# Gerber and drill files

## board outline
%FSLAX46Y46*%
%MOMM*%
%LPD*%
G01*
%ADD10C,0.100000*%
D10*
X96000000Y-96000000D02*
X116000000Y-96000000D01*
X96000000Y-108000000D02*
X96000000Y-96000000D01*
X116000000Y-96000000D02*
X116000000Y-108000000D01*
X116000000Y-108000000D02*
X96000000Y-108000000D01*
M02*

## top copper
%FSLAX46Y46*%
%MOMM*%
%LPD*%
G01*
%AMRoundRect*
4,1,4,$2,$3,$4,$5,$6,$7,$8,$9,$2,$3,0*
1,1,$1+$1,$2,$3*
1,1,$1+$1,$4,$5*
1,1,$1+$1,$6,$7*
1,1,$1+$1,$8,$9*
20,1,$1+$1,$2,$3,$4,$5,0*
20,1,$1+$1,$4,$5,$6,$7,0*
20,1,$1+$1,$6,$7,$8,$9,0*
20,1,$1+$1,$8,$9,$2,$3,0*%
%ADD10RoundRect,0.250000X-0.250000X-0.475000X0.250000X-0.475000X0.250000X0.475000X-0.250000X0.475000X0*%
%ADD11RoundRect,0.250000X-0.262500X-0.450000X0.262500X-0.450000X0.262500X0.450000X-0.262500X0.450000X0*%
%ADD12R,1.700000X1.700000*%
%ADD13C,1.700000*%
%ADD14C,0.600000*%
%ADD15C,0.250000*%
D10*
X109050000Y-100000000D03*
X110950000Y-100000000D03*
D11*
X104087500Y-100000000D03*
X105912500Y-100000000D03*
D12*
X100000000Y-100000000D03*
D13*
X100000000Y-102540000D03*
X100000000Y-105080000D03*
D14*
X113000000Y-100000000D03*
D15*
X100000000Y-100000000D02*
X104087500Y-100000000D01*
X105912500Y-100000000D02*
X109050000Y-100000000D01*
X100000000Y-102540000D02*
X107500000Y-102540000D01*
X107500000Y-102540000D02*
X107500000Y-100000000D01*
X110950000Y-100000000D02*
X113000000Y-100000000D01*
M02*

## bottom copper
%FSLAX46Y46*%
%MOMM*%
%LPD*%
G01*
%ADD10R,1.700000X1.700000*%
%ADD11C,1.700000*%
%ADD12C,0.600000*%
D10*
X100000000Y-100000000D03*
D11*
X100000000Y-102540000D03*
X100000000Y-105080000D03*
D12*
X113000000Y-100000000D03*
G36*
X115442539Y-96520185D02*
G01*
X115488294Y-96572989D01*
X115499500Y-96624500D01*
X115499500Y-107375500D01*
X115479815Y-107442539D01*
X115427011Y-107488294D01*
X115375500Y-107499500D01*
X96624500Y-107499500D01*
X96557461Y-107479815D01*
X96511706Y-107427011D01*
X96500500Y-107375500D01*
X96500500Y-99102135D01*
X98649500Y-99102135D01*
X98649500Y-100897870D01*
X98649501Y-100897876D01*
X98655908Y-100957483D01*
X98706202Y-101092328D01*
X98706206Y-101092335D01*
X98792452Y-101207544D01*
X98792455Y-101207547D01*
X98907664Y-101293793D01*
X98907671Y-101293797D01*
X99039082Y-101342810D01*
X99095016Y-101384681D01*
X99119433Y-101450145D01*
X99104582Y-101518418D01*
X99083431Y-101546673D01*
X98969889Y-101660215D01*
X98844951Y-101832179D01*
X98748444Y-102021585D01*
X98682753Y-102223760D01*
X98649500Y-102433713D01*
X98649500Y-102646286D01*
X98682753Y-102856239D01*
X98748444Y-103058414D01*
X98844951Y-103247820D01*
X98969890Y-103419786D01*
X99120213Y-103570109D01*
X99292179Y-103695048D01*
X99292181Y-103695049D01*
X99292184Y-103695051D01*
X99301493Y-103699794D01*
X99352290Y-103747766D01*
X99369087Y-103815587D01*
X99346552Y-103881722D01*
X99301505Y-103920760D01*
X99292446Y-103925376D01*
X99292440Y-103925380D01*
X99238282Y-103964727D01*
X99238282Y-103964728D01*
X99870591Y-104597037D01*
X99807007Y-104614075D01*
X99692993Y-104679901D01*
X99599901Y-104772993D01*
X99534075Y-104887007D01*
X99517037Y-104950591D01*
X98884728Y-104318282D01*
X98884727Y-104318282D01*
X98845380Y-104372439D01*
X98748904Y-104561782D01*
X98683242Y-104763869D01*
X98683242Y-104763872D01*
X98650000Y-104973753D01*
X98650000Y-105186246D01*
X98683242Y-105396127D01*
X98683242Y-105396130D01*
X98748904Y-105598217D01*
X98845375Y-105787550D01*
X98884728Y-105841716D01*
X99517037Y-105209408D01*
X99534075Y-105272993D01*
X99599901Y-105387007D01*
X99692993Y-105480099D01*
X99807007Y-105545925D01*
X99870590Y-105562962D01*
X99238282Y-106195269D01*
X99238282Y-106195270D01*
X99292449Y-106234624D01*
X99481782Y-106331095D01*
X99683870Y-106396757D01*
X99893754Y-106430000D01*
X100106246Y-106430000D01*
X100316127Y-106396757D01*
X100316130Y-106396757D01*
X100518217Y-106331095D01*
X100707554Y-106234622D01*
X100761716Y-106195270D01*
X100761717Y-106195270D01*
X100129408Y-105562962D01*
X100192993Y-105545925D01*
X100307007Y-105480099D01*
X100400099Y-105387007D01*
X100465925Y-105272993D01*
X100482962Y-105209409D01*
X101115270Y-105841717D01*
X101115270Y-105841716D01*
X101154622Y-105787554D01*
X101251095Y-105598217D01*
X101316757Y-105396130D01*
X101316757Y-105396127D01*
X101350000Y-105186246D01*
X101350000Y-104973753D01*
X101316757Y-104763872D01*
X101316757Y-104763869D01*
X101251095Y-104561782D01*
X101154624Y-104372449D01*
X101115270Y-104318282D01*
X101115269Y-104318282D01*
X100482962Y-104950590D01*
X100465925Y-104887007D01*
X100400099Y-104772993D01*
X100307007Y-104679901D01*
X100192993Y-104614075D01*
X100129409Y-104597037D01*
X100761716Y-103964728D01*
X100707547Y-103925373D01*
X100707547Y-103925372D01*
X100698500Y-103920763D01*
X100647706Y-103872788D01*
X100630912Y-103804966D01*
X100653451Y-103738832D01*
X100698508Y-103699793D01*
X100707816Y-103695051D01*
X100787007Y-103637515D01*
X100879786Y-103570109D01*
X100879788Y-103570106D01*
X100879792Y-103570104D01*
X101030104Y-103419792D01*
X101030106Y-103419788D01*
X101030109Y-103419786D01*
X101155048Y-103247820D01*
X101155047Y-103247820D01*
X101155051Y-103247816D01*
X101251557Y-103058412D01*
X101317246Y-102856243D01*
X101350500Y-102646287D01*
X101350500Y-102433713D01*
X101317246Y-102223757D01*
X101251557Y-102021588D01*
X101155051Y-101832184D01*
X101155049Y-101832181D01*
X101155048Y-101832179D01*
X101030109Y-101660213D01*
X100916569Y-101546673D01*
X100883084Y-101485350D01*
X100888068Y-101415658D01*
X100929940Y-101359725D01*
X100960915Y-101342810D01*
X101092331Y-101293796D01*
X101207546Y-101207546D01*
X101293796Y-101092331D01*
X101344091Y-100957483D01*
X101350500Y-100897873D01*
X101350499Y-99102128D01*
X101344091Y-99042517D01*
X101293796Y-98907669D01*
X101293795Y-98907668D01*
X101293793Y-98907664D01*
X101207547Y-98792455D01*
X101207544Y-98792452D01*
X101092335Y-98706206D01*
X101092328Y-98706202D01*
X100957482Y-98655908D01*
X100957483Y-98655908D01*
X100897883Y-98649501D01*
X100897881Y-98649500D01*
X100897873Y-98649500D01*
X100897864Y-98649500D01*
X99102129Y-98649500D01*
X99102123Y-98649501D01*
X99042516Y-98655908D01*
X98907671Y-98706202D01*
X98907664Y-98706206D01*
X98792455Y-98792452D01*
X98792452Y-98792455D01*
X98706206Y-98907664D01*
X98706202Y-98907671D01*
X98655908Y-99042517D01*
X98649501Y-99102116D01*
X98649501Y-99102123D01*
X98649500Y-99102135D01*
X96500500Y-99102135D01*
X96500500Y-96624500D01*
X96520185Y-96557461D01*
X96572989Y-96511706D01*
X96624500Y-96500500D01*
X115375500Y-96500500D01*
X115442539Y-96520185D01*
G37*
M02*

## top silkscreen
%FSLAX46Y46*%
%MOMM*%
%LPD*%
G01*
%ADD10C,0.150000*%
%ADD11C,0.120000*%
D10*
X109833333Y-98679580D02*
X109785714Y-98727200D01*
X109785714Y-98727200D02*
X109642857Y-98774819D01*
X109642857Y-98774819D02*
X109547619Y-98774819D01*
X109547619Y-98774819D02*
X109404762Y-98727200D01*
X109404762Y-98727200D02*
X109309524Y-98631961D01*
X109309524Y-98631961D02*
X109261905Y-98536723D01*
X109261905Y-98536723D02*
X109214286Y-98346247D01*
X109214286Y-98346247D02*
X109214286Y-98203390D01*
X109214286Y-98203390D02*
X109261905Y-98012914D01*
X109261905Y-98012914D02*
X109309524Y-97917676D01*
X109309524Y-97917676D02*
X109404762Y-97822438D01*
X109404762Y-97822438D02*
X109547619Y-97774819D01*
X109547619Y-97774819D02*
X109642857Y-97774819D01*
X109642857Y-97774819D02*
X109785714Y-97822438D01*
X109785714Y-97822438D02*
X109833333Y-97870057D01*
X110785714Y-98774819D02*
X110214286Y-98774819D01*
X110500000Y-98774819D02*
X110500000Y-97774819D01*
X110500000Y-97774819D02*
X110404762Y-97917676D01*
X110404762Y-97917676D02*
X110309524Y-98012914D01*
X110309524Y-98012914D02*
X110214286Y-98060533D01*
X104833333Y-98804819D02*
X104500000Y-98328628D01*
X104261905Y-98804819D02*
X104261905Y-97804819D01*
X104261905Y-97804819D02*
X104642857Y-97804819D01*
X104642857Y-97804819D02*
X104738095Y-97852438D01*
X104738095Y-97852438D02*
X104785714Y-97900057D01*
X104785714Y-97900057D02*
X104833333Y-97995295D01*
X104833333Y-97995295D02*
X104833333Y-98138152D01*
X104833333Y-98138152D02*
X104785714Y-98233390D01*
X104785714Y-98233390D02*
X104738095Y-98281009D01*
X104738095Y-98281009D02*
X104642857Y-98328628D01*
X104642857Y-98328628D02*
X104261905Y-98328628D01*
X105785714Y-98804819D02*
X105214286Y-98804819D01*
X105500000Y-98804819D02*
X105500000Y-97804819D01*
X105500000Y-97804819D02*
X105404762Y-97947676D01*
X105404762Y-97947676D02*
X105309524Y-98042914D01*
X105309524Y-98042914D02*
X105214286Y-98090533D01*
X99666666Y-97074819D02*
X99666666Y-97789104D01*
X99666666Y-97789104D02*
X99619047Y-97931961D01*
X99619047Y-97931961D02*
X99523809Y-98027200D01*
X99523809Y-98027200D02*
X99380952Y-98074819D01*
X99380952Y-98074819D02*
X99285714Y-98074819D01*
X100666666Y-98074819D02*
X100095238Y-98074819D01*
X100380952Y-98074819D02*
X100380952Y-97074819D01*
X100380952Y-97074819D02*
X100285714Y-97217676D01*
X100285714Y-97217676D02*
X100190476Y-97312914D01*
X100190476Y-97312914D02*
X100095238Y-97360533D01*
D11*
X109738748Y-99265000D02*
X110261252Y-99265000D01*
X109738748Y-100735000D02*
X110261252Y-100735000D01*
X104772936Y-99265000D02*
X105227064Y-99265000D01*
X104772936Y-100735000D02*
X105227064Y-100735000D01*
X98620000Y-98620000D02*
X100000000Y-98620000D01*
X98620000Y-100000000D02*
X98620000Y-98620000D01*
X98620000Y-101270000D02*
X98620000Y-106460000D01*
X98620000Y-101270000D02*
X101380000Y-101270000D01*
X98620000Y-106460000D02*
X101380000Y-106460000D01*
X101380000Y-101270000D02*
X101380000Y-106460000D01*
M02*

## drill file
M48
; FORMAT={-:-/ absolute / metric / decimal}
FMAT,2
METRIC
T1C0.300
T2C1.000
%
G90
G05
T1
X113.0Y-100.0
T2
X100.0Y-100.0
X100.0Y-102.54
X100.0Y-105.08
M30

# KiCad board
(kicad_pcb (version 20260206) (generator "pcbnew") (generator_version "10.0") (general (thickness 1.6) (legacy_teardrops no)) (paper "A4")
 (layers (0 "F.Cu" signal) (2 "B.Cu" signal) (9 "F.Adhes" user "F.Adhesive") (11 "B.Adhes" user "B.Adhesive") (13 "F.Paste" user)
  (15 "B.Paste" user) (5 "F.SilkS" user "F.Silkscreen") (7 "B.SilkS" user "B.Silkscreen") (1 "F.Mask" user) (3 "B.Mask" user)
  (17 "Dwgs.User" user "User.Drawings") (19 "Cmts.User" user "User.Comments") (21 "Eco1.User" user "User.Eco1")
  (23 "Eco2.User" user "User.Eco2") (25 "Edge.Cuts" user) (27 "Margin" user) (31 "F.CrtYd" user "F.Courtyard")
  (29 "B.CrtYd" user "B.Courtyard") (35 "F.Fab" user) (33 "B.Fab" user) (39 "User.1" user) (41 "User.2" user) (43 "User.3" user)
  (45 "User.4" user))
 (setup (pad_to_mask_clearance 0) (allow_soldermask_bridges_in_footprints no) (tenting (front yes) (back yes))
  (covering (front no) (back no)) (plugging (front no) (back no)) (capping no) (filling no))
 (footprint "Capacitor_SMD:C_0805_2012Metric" (layer "F.Cu") (at 110 100)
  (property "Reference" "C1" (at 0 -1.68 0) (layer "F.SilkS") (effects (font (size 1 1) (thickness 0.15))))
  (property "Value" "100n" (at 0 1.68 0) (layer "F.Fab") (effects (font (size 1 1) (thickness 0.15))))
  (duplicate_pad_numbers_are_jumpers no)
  (fp_line (start -0.261252 -0.735) (end 0.261252 -0.735) (stroke (width 0.12) (type solid)) (layer "F.SilkS"))
  (fp_line (start -0.261252 0.735) (end 0.261252 0.735) (stroke (width 0.12) (type solid)) (layer "F.SilkS"))
  (pad "1" smd roundrect (at -0.95 0) (size 1 1.45) (layers "F.Cu" "F.Mask" "F.Paste") (roundrect_rratio 0.25) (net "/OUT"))
  (pad "2" smd roundrect (at 0.95 0) (size 1 1.45) (layers "F.Cu" "F.Mask" "F.Paste") (roundrect_rratio 0.25) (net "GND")))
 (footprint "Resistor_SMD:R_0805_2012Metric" (layer "F.Cu") (at 105 100)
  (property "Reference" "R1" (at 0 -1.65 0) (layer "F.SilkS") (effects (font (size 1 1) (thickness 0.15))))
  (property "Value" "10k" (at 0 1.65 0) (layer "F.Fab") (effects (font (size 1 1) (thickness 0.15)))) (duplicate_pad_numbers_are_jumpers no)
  (fp_line (start -0.227064 -0.735) (end 0.227064 -0.735) (stroke (width 0.12) (type solid)) (layer "F.SilkS"))
  (fp_line (start -0.227064 0.735) (end 0.227064 0.735) (stroke (width 0.12) (type solid)) (layer "F.SilkS"))
  (pad "1" smd roundrect (at -0.9125 0) (size 1.025 1.4) (layers "F.Cu" "F.Mask" "F.Paste") (roundrect_rratio 0.243902) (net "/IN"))
  (pad "2" smd roundrect (at 0.9125 0) (size 1.025 1.4) (layers "F.Cu" "F.Mask" "F.Paste") (roundrect_rratio 0.243902) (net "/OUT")))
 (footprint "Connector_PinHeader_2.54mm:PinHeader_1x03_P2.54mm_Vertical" (layer "F.Cu") (at 100 100)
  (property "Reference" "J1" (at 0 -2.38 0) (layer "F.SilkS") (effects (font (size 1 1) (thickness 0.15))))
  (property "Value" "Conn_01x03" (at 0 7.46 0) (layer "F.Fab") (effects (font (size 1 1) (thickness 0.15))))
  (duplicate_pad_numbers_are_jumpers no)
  (fp_line (start -1.38 -1.38) (end 0 -1.38) (stroke (width 0.12) (type solid)) (layer "F.SilkS"))
  (fp_line (start -1.38 0) (end -1.38 -1.38) (stroke (width 0.12) (type solid)) (layer "F.SilkS"))
  (fp_line (start -1.38 1.27) (end -1.38 6.46) (stroke (width 0.12) (type solid)) (layer "F.SilkS"))
  (fp_line (start -1.38 1.27) (end 1.38 1.27) (stroke (width 0.12) (type solid)) (layer "F.SilkS"))
  (fp_line (start -1.38 6.46) (end 1.38 6.46) (stroke (width 0.12) (type solid)) (layer "F.SilkS"))
  (fp_line (start 1.38 1.27) (end 1.38 6.46) (stroke (width 0.12) (type solid)) (layer "F.SilkS"))
  (pad "1" thru_hole rect (at 0 0) (size 1.7 1.7) (drill 1) (layers "*.Cu" "*.Mask") (remove_unused_layers no) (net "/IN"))
  (pad "2" thru_hole circle (at 0 2.54) (size 1.7 1.7) (drill 1) (layers "*.Cu" "*.Mask") (remove_unused_layers no) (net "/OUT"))
  (pad "3" thru_hole circle (at 0 5.08) (size 1.7 1.7) (drill 1) (layers "*.Cu" "*.Mask") (remove_unused_layers no) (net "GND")))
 (gr_line (start 96 96) (end 116 96) (stroke (width 0.1) (type default)) (layer "Edge.Cuts"))
 (gr_line (start 96 108) (end 96 96) (stroke (width 0.1) (type default)) (layer "Edge.Cuts"))
 (gr_line (start 116 96) (end 116 108) (stroke (width 0.1) (type default)) (layer "Edge.Cuts"))
 (gr_line (start 116 108) (end 96 108) (stroke (width 0.1) (type default)) (layer "Edge.Cuts"))
 (segment (start 100 100) (end 104.0875 100) (width 0.25) (layer "F.Cu") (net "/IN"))
 (segment (start 105.9125 100) (end 109.05 100) (width 0.25) (layer "F.Cu") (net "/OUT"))
 (segment (start 100 102.54) (end 107.5 102.54) (width 0.25) (layer "F.Cu") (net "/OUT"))
 (segment (start 107.5 102.54) (end 107.5 100) (width 0.25) (layer "F.Cu") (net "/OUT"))
 (segment (start 110.95 100) (end 113 100) (width 0.25) (layer "F.Cu") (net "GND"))
 (via (at 113 100) (size 0.6) (drill 0.3) (layers "F.Cu" "B.Cu") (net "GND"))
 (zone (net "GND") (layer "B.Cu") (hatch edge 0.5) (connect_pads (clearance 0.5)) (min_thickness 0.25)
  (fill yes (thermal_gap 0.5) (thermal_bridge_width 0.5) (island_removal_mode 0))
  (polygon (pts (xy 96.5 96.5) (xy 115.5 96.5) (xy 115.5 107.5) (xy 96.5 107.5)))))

